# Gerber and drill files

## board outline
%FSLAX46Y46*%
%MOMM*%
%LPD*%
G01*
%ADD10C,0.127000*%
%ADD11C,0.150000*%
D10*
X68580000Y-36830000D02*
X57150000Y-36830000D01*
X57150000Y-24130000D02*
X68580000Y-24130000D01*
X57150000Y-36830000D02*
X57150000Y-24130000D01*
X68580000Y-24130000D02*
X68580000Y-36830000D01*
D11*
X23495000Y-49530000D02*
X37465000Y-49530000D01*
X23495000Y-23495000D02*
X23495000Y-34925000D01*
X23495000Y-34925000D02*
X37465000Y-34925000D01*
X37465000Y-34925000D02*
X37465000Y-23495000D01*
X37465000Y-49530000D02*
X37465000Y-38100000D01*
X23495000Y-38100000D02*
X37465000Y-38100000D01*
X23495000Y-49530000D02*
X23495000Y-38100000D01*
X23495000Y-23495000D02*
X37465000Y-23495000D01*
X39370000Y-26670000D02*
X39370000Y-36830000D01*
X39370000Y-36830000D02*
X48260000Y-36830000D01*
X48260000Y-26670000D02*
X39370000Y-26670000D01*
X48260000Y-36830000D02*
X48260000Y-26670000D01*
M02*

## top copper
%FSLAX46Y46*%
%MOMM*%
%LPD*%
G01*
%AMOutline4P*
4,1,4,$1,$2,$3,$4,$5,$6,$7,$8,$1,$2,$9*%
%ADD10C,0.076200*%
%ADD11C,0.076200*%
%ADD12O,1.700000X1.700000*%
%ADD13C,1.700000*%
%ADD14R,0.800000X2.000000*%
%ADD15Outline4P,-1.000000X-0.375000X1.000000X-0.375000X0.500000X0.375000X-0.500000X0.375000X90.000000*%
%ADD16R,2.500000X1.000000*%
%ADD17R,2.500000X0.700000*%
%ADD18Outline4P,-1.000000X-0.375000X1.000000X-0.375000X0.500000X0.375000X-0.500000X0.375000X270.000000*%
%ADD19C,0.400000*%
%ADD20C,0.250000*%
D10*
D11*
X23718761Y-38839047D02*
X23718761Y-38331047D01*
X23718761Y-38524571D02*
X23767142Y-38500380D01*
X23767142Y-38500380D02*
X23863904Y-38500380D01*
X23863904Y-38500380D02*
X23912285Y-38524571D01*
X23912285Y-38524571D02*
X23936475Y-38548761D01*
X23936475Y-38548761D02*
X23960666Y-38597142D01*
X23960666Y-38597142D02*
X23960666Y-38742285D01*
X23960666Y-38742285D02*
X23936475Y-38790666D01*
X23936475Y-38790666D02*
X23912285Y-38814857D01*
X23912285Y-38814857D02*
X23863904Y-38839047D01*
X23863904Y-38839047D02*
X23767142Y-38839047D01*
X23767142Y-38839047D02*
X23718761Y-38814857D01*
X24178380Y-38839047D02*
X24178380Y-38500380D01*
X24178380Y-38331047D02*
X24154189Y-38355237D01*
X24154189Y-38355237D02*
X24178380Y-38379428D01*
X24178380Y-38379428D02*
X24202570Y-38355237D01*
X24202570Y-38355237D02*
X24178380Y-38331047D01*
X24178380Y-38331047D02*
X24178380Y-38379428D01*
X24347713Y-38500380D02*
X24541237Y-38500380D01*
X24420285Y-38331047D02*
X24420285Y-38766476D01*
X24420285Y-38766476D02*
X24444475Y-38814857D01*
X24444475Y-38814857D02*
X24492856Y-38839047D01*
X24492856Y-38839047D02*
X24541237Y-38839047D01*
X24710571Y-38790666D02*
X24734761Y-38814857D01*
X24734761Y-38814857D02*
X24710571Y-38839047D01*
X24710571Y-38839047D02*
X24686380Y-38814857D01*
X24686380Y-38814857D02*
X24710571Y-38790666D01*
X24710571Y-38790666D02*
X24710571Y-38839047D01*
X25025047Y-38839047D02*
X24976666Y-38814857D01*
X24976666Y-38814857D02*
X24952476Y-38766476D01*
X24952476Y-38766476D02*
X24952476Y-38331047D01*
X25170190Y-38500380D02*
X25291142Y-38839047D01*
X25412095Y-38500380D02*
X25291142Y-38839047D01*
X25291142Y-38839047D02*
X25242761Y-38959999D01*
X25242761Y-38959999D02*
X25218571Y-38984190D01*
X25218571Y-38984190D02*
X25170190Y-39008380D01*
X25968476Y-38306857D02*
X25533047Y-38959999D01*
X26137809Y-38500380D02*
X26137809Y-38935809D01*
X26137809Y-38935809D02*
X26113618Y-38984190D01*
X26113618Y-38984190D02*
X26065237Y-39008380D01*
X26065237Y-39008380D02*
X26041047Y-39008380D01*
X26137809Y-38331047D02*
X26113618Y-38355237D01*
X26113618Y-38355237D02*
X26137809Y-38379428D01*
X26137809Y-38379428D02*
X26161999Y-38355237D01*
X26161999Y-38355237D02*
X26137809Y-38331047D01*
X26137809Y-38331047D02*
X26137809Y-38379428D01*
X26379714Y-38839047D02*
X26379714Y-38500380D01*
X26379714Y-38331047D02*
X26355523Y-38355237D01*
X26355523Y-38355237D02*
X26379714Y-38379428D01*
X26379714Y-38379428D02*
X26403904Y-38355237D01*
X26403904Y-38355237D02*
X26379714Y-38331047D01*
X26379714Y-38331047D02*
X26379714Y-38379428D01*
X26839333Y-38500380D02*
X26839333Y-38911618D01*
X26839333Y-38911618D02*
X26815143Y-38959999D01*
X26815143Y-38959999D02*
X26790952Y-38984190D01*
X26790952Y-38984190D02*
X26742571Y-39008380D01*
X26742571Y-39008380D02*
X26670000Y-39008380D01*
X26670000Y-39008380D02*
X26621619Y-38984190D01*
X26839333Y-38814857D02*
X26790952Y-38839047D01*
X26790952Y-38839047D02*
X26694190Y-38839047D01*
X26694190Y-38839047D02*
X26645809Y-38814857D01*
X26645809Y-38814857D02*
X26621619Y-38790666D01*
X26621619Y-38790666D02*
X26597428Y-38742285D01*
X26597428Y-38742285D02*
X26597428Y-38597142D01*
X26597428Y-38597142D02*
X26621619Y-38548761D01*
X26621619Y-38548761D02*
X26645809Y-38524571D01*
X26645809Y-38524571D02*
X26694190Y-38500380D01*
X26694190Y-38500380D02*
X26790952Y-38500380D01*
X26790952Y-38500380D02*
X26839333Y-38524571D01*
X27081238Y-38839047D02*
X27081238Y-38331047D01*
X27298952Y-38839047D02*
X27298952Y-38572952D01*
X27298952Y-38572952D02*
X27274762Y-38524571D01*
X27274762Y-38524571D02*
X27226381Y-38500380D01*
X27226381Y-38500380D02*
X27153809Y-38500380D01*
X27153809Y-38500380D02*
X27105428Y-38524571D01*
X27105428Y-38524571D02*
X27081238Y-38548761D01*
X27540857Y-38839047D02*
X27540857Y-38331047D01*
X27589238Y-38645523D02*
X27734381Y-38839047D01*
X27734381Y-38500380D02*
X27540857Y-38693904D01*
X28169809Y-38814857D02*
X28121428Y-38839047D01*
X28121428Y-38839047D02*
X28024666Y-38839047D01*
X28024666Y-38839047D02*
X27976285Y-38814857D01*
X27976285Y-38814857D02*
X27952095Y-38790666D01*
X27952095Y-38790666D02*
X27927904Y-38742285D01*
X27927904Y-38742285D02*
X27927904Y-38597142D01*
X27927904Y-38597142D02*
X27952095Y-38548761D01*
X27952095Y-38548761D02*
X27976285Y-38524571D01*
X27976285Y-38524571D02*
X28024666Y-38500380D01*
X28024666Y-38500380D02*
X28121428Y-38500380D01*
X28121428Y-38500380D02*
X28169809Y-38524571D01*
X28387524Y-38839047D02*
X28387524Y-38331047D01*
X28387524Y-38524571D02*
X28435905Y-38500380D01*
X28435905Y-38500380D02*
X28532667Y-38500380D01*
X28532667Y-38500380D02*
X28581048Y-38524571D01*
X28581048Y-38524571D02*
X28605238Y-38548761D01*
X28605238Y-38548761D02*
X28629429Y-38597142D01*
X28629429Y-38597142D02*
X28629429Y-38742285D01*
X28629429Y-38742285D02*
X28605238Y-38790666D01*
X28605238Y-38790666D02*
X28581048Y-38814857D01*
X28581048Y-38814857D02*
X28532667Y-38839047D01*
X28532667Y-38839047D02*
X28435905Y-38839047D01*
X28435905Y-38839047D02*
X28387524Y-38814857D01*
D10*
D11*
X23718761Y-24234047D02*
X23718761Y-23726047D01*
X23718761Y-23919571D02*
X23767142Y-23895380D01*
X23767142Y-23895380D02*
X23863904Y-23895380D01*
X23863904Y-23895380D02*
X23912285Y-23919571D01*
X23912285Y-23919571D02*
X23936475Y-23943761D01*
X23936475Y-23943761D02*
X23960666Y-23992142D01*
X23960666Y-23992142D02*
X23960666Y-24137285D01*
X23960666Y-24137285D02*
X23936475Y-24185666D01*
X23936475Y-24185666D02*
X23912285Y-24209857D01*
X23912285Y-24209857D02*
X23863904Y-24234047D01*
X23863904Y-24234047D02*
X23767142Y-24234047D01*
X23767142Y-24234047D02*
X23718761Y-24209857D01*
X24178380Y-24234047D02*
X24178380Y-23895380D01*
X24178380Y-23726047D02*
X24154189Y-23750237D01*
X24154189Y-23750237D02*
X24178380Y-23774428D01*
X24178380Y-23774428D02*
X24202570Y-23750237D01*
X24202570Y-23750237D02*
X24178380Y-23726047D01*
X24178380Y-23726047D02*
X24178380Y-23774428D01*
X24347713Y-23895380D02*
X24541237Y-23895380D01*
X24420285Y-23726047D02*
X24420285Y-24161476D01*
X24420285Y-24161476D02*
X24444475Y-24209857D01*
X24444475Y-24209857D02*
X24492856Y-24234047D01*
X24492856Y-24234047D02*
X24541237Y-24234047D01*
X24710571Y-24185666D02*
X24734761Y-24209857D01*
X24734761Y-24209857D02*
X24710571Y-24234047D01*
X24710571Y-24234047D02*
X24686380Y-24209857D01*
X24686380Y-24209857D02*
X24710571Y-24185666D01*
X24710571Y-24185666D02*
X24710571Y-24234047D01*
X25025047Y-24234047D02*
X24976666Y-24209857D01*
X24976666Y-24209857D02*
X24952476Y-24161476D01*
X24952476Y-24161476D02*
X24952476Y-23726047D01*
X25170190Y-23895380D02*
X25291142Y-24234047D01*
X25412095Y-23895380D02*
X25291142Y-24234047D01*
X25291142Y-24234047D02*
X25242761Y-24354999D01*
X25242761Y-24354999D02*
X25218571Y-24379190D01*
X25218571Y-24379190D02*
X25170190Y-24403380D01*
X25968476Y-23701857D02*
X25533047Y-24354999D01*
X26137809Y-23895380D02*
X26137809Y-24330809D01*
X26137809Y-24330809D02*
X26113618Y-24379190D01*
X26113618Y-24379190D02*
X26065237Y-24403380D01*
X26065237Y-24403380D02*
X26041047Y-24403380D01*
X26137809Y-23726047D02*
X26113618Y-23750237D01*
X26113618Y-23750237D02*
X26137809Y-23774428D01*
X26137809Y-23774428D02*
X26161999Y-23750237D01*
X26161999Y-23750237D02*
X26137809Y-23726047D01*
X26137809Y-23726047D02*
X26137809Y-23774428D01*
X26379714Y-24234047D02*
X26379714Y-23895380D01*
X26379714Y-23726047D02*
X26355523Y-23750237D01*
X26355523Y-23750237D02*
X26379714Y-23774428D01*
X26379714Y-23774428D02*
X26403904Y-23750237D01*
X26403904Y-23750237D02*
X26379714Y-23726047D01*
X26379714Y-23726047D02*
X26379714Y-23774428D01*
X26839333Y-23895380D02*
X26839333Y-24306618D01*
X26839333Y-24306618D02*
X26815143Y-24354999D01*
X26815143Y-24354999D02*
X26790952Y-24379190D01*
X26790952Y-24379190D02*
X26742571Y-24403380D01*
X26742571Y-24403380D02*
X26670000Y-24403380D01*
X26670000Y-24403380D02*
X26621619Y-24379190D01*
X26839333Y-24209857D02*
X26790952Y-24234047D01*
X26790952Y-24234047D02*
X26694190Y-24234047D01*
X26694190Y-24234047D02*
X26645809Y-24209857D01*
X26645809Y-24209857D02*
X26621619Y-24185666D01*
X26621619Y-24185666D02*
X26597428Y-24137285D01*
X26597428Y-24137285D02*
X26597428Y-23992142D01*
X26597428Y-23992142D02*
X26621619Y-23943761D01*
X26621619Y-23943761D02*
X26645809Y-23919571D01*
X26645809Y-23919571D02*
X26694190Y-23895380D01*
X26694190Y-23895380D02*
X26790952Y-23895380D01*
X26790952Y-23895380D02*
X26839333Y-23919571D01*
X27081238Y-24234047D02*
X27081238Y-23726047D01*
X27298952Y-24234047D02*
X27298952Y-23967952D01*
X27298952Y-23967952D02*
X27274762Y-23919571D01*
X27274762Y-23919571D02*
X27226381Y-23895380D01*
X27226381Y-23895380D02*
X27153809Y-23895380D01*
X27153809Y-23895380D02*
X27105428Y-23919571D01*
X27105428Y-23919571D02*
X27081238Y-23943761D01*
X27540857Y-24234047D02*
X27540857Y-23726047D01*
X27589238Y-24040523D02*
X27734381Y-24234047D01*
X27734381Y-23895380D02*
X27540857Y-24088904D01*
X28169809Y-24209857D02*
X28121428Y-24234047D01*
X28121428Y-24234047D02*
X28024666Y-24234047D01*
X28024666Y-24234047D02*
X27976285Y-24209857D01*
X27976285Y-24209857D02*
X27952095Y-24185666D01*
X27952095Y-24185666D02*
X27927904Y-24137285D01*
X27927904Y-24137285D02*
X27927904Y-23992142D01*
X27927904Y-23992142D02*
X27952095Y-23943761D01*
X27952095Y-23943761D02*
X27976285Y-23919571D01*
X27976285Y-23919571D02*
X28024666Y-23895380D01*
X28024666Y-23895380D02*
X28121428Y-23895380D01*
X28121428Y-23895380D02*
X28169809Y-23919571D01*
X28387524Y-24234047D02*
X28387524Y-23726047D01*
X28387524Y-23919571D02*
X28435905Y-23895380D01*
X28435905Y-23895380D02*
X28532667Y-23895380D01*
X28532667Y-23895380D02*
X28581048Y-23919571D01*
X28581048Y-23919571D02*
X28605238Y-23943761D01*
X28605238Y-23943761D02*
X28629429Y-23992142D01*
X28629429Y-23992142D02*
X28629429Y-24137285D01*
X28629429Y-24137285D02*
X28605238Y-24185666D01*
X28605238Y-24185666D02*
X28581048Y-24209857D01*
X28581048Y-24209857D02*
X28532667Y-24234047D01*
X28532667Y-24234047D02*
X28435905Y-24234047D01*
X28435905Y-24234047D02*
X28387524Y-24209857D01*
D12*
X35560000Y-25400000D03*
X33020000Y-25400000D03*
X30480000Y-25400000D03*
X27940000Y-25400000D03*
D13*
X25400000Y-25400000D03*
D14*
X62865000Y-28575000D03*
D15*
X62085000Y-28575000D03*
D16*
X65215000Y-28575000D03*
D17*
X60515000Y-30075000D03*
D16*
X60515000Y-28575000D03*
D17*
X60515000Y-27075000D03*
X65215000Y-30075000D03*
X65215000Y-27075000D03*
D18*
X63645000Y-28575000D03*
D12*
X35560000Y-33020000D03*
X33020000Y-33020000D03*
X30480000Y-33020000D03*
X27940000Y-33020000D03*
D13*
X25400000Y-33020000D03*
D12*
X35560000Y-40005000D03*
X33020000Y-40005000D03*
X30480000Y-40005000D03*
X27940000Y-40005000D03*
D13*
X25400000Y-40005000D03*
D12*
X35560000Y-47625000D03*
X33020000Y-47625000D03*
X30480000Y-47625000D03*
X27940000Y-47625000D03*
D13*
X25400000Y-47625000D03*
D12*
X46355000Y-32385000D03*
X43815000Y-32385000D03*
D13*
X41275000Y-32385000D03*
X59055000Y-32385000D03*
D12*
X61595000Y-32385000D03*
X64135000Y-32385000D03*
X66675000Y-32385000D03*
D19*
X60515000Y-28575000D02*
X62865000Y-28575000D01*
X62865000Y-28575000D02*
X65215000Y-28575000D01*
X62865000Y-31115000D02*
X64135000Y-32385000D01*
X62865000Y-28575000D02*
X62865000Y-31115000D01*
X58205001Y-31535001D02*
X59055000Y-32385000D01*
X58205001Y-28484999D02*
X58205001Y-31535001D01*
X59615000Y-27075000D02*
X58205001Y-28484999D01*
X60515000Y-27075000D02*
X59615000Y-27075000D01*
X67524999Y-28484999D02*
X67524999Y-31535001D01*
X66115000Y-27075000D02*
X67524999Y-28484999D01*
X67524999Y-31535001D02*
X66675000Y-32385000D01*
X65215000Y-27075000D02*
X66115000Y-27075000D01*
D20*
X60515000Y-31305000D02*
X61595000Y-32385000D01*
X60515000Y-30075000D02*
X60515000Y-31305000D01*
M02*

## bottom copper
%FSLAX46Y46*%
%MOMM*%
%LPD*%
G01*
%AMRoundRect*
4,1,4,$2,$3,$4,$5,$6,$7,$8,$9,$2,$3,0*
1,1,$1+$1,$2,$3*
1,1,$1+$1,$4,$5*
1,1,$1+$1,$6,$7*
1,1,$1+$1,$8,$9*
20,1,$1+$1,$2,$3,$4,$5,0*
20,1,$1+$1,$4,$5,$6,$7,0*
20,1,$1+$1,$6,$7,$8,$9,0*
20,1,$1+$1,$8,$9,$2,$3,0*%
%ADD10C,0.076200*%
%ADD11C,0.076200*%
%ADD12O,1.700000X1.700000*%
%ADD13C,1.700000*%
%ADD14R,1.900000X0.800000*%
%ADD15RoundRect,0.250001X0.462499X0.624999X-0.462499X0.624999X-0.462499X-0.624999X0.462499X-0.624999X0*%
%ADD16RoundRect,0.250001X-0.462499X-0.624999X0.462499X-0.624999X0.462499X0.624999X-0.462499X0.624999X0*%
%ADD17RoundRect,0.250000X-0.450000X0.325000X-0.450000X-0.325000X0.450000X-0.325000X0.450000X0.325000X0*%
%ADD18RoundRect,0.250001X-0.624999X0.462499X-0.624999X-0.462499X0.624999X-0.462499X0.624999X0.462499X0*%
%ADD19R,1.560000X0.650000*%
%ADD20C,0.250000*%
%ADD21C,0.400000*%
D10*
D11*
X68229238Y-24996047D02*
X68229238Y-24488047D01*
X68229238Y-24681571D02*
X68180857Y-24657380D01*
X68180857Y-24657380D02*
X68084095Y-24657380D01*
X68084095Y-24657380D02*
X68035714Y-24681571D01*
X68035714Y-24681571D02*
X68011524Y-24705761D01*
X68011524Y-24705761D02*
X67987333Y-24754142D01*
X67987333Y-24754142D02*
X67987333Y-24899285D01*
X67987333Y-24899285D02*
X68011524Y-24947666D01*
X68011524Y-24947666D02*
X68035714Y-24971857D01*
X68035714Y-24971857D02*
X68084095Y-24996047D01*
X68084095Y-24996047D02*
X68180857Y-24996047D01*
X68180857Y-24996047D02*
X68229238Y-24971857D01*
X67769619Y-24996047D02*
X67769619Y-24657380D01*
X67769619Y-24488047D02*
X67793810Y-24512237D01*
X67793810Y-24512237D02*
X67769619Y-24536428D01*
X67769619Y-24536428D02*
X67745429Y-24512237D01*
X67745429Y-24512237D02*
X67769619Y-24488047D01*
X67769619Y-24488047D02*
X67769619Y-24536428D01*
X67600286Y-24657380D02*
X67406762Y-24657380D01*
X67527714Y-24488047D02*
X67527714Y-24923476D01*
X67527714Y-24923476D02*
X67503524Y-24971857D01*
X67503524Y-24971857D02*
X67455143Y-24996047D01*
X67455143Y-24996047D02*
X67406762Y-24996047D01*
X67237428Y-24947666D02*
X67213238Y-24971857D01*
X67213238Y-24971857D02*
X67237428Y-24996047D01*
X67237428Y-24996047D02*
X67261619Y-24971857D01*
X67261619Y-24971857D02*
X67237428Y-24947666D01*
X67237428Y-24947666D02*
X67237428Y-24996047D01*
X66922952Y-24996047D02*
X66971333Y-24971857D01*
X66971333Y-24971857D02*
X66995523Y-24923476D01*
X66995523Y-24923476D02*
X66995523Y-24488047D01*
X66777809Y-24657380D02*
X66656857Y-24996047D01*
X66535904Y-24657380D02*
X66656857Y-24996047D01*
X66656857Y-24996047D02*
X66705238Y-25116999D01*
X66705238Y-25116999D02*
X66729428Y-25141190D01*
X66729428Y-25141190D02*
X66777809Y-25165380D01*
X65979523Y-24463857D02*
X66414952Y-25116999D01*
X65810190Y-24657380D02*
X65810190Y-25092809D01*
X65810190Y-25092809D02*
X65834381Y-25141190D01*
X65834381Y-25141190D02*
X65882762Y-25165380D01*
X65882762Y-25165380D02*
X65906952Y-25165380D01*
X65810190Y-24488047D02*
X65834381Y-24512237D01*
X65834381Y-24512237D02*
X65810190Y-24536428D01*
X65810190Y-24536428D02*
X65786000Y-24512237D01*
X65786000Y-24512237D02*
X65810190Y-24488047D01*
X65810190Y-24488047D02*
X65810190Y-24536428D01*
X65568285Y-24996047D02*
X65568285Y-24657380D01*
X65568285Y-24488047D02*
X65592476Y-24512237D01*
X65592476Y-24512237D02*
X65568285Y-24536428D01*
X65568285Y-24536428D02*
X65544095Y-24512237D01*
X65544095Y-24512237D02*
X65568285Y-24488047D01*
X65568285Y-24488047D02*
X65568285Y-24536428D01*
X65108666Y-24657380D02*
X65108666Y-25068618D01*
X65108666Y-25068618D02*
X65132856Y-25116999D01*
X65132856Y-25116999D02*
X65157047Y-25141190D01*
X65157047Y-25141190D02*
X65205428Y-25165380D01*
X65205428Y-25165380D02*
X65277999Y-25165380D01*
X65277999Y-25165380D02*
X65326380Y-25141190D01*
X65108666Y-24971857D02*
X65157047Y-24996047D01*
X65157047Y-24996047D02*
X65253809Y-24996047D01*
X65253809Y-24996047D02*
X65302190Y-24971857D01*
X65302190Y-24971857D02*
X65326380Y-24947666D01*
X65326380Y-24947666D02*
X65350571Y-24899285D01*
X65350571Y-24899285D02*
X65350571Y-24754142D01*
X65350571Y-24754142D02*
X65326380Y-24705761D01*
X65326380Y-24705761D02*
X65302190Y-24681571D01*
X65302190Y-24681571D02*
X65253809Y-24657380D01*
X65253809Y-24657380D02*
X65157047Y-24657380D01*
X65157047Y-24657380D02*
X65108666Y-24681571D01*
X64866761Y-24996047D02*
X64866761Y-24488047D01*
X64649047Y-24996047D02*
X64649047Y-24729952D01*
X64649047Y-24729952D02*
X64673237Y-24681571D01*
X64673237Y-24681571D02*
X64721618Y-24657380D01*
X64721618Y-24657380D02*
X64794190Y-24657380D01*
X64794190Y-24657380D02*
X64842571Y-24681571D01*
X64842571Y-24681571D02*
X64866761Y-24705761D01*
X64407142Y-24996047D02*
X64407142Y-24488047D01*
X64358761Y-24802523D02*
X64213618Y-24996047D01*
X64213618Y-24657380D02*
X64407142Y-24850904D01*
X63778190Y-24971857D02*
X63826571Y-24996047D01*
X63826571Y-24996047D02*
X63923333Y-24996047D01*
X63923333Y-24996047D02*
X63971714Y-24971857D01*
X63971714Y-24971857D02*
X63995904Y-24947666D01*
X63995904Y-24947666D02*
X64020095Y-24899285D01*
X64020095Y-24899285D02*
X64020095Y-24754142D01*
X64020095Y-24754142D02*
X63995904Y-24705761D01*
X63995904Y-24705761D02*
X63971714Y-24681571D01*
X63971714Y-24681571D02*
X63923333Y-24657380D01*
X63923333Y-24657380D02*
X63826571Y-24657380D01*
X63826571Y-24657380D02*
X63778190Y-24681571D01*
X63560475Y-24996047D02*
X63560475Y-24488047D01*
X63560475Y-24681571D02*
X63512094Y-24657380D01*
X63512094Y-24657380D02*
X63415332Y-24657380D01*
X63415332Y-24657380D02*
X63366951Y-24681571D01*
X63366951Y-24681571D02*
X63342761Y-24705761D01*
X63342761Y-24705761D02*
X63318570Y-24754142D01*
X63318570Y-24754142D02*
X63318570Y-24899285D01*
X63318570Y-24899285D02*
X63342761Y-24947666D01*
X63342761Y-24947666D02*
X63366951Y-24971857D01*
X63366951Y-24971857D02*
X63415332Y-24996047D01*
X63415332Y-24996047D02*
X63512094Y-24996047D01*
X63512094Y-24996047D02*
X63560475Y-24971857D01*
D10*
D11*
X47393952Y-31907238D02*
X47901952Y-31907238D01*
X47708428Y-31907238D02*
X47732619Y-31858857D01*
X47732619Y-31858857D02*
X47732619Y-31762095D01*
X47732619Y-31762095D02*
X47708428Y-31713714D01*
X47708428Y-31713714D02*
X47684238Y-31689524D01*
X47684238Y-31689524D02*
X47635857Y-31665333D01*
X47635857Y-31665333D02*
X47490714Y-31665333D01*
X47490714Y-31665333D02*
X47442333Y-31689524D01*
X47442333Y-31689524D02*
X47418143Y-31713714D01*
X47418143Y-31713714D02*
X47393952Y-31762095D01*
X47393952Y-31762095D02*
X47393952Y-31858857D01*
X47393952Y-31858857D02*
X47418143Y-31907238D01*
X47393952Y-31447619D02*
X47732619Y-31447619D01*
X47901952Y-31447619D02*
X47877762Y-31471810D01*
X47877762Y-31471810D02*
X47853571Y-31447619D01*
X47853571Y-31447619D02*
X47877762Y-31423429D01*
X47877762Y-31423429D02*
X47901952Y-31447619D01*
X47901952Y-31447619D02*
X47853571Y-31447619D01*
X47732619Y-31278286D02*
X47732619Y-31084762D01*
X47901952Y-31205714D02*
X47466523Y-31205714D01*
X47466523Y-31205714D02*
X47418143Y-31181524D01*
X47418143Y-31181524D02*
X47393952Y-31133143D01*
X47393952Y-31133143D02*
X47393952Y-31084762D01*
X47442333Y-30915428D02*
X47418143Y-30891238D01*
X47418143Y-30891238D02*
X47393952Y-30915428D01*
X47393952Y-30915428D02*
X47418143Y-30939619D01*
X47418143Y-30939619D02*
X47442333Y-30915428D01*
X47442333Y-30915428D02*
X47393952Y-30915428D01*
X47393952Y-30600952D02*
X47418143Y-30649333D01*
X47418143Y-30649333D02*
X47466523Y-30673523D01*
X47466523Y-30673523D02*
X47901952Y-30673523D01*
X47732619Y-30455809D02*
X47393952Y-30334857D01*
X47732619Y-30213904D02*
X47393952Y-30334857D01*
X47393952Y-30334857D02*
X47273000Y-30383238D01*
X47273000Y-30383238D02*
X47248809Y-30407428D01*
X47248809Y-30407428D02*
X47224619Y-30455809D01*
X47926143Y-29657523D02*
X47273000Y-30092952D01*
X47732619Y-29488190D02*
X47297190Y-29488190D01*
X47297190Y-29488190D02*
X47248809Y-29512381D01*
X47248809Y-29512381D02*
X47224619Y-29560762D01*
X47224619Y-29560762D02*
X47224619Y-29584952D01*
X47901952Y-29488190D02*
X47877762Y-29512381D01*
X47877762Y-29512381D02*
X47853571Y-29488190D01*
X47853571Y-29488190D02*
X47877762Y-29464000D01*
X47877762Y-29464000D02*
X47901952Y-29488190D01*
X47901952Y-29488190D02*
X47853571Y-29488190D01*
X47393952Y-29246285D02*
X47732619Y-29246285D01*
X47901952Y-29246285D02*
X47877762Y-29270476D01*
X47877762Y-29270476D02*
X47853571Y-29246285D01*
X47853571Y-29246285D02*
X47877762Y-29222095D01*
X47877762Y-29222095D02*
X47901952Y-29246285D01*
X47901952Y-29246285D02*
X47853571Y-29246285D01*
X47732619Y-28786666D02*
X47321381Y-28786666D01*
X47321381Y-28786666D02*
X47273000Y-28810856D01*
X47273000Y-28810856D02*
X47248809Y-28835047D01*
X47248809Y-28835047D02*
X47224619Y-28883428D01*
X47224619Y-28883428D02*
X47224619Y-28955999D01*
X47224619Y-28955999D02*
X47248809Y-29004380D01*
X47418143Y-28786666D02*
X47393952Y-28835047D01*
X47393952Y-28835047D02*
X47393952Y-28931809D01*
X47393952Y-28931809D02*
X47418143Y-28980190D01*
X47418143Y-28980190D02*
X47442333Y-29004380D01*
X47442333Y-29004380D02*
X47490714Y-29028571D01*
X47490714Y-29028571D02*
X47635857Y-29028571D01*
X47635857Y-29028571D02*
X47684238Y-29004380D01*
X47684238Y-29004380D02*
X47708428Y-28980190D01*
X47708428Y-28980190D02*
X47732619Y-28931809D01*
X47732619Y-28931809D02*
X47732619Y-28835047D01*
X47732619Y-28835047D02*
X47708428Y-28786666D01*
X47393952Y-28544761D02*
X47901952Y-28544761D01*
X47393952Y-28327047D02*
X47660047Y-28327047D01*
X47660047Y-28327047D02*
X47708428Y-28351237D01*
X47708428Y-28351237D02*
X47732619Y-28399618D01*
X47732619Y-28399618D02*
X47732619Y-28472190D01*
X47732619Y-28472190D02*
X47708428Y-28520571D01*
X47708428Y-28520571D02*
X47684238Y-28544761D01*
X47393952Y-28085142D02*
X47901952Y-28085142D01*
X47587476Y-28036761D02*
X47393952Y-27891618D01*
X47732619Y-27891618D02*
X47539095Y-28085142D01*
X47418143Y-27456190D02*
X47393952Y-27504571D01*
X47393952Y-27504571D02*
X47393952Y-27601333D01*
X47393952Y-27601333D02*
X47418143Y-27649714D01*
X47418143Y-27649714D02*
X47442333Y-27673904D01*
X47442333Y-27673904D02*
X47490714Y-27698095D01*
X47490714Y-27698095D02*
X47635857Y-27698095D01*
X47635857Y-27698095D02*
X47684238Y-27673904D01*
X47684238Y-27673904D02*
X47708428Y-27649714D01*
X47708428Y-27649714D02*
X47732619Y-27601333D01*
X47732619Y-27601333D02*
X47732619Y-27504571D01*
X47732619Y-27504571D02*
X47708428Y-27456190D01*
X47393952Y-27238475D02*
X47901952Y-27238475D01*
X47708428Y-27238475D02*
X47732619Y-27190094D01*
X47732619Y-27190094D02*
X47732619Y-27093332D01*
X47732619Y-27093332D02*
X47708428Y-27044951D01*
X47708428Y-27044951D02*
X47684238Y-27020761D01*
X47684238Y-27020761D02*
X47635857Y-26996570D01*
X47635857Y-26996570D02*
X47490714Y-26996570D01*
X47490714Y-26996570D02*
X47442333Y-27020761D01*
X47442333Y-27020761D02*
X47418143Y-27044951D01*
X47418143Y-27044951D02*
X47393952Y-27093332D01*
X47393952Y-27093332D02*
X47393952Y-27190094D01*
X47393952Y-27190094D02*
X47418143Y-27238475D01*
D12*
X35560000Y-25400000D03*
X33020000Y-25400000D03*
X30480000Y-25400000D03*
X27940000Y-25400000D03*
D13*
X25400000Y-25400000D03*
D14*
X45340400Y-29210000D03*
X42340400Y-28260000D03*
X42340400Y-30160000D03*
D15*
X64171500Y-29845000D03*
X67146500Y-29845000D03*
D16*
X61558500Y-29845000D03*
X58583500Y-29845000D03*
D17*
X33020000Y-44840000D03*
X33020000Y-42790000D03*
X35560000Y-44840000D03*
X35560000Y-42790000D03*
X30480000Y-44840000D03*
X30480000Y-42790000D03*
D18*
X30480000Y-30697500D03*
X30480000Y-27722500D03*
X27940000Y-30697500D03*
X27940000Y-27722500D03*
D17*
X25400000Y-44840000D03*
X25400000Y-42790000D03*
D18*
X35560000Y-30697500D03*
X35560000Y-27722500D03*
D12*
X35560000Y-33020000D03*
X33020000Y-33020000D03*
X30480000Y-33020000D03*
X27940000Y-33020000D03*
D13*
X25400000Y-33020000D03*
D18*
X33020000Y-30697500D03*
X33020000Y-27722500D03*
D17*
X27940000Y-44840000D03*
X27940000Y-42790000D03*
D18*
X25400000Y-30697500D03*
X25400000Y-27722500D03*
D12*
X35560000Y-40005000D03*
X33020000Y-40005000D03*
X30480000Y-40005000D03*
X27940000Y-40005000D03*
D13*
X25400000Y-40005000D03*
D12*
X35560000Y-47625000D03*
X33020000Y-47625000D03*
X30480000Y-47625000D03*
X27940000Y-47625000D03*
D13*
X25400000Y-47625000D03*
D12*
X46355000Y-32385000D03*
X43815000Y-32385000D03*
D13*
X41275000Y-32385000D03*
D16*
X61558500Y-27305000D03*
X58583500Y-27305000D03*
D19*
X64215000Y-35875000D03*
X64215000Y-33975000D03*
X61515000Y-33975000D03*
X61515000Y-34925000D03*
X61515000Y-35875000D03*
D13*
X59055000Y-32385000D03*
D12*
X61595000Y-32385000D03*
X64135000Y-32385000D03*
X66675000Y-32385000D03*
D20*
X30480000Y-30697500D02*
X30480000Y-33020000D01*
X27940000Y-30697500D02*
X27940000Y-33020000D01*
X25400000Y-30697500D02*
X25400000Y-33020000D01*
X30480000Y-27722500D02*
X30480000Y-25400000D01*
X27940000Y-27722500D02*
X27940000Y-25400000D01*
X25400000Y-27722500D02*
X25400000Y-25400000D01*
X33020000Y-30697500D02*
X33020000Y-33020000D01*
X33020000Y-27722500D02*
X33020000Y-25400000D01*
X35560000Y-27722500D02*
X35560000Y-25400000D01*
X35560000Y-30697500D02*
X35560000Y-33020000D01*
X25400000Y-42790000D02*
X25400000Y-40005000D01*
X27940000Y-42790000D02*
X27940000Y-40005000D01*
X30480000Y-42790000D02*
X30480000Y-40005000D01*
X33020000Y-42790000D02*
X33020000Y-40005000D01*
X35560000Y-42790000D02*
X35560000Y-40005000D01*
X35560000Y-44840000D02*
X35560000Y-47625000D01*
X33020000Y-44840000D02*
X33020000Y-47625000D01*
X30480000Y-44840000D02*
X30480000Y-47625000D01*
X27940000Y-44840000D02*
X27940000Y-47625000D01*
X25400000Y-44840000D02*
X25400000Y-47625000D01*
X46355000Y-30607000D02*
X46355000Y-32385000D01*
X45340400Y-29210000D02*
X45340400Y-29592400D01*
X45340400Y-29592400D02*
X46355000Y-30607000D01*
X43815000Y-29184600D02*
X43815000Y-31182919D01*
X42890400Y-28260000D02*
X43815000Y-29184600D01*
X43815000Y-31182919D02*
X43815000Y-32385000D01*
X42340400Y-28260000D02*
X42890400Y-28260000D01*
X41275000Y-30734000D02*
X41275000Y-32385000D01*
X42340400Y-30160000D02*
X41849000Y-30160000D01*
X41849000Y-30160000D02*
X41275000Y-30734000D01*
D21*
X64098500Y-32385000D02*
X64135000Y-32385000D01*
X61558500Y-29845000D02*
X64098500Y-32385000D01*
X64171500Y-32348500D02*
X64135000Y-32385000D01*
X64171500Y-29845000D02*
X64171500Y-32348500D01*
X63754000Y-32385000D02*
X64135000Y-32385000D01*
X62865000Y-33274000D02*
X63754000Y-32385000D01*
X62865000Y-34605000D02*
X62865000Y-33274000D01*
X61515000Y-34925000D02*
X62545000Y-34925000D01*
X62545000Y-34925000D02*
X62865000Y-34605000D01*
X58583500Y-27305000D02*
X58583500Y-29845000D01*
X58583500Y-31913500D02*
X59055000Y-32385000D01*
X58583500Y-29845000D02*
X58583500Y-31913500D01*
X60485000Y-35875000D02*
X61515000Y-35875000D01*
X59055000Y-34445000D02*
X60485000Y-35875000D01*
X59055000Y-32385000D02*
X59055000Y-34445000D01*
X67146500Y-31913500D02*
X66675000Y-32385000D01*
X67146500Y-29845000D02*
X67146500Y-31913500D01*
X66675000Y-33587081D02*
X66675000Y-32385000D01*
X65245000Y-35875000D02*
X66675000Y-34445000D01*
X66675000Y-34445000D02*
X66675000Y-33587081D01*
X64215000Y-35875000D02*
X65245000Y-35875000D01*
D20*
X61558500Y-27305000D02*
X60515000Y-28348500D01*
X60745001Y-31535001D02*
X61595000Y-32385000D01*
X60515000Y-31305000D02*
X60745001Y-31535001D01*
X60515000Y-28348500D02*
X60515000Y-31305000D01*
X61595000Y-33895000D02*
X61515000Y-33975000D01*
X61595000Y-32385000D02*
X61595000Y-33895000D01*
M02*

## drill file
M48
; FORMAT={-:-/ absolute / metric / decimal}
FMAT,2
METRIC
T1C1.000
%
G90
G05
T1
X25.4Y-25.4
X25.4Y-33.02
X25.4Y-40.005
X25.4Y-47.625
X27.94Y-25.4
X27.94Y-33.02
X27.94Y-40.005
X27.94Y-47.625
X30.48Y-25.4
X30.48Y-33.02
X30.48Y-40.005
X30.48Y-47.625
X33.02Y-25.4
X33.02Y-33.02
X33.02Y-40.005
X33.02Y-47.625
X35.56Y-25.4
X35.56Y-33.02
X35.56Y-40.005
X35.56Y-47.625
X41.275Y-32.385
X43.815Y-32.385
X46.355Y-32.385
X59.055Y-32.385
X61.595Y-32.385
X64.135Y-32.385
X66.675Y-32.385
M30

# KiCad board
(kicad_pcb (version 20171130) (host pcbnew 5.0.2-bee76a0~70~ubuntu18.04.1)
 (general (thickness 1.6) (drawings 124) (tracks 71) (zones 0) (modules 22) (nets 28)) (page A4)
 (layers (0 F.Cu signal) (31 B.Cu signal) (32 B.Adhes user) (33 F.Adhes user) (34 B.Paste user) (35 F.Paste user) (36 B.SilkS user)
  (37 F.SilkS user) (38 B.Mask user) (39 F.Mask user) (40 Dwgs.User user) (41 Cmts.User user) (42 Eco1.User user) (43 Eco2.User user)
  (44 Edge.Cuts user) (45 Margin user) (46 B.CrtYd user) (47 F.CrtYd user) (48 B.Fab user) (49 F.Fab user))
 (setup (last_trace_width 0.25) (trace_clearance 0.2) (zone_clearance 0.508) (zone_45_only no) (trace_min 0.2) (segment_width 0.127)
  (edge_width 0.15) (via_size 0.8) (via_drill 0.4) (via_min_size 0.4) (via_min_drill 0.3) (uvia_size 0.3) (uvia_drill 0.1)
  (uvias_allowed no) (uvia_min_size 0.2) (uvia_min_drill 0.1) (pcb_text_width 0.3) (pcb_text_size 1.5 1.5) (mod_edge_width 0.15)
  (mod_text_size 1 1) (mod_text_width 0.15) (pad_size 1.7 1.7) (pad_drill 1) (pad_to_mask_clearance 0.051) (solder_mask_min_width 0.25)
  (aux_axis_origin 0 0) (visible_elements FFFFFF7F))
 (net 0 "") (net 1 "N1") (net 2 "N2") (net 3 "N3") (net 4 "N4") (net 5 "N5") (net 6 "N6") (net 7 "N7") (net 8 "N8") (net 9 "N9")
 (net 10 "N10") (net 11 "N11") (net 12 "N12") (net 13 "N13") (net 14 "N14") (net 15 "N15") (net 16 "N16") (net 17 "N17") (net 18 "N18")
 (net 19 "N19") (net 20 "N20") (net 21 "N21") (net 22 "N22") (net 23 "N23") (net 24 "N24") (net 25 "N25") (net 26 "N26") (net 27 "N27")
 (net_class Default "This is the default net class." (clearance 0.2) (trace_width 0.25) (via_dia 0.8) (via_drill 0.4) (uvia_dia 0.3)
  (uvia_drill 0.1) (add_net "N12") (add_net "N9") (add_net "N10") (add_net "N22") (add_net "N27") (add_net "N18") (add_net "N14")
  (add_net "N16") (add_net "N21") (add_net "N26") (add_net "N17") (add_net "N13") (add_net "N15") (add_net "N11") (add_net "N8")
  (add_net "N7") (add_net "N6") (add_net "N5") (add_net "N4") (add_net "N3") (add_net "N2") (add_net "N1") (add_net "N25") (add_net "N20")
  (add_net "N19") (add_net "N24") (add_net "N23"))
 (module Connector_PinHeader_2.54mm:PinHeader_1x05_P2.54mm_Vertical (layer B.Cu) (at 25.4 25.4 270)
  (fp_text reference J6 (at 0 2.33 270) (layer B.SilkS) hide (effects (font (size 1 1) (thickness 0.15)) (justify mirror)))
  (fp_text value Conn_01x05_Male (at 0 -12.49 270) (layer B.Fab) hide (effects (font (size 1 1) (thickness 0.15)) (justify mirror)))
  (pad 5 thru_hole oval (at 0 -10.16 270) (size 1.7 1.7) (drill 1) (layers *.Cu *.Mask) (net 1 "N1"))
  (pad 4 thru_hole oval (at 0 -7.62 270) (size 1.7 1.7) (drill 1) (layers *.Cu *.Mask) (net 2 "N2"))
  (pad 3 thru_hole oval (at 0 -5.08 270) (size 1.7 1.7) (drill 1) (layers *.Cu *.Mask) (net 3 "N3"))
  (pad 2 thru_hole oval (at 0 -2.54 270) (size 1.7 1.7) (drill 1) (layers *.Cu *.Mask) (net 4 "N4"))
  (pad 1 thru_hole circle (at 0 0 270) (size 1.7 1.7) (drill 1) (layers *.Cu *.Mask) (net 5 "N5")))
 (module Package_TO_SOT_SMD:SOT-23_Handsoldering (layer B.Cu) (at 43.8404 29.21)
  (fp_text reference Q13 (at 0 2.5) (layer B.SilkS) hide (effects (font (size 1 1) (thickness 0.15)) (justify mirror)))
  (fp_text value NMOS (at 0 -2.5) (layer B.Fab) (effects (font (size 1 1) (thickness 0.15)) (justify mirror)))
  (pad 3 smd rect (at 1.5 0) (size 1.9 0.8) (layers B.Cu B.Paste B.Mask) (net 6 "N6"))
  (pad 2 smd rect (at -1.5 -0.95) (size 1.9 0.8) (layers B.Cu B.Paste B.Mask) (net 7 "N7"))
  (pad 1 smd rect (at -1.5 0.95) (size 1.9 0.8) (layers B.Cu B.Paste B.Mask) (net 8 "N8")))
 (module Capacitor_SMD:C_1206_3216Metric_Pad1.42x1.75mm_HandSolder (layer B.Cu) (at 65.659 29.845 180)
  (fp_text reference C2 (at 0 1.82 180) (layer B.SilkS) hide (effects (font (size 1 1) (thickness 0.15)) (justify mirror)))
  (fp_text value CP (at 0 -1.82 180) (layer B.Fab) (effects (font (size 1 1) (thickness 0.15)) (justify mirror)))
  (pad 2 smd roundrect (at 1.4875 0 180) (size 1.425 1.75) (layers B.Cu B.Paste B.Mask) (roundrect_rratio 0.175439) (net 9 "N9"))
  (pad 1 smd roundrect (at -1.4875 0 180) (size 1.425 1.75) (layers B.Cu B.Paste B.Mask) (roundrect_rratio 0.175439) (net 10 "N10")))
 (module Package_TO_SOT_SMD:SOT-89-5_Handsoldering (layer F.Cu) (at 62.865 28.575)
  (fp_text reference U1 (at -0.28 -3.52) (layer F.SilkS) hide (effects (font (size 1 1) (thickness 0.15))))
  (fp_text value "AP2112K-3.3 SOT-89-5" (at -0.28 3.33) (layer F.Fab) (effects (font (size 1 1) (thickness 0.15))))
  (pad 2 smd rect (at 0 0 270) (size 2 0.8) (layers F.Cu F.Paste F.Mask) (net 9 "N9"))
  (pad 2 smd trapezoid (at -0.78 0 90) (size 1.5 0.75) (rect_delta 0 0.5) (layers F.Cu F.Paste F.Mask) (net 9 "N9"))
  (pad 2 smd rect (at 2.35 0 270) (size 1 2.5) (layers F.Cu F.Paste F.Mask) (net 9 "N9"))
  (pad 3 smd rect (at -2.35 1.5 270) (size 0.7 2.5) (layers F.Cu F.Paste F.Mask) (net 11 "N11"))
  (pad 2 smd rect (at -2.35 0 270) (size 1 2.5) (layers F.Cu F.Paste F.Mask) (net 9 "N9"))
  (pad 1 smd rect (at -2.35 -1.5 270) (size 0.7 2.5) (layers F.Cu F.Paste F.Mask) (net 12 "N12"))
  (pad 4 smd rect (at 2.35 1.5 270) (size 0.7 2.5) (layers F.Cu F.Paste F.Mask))
  (pad 5 smd rect (at 2.35 -1.5 270) (size 0.7 2.5) (layers F.Cu F.Paste F.Mask) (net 10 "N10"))
  (pad 2 smd trapezoid (at 0.78 0 270) (size 1.5 0.75) (rect_delta 0 0.5) (layers F.Cu F.Paste F.Mask) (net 9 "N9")))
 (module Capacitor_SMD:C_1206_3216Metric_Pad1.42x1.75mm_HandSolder (layer B.Cu) (at 60.071 29.845)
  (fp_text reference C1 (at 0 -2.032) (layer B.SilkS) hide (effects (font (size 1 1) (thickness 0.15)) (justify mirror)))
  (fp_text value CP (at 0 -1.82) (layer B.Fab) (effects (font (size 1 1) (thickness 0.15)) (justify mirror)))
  (pad 2 smd roundrect (at 1.4875 0) (size 1.425 1.75) (layers B.Cu B.Paste B.Mask) (roundrect_rratio 0.175439) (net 9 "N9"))
  (pad 1 smd roundrect (at -1.4875 0) (size 1.425 1.75) (layers B.Cu B.Paste B.Mask) (roundrect_rratio 0.175439) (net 12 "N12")))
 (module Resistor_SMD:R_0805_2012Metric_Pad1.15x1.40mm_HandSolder (layer B.Cu) (at 33.02 43.815 270)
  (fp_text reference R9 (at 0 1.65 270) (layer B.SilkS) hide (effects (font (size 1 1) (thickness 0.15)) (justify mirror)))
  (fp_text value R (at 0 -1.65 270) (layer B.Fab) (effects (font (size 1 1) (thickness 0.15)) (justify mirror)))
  (pad 2 smd roundrect (at 1.025 0 270) (size 1.15 1.4) (layers B.Cu B.Paste B.Mask) (roundrect_rratio 0.217391) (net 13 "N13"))
  (pad 1 smd roundrect (at -1.025 0 270) (size 1.15 1.4) (layers B.Cu B.Paste B.Mask) (roundrect_rratio 0.217391) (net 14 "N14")))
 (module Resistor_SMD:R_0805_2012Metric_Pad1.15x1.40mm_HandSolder (layer B.Cu) (at 35.56 43.815 270)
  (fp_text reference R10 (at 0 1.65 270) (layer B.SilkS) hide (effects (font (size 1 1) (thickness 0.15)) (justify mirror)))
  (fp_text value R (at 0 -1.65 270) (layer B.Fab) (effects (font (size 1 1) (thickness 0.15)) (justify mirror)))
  (pad 2 smd roundrect (at 1.025 0 270) (size 1.15 1.4) (layers B.Cu B.Paste B.Mask) (roundrect_rratio 0.217391) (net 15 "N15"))
  (pad 1 smd roundrect (at -1.025 0 270) (size 1.15 1.4) (layers B.Cu B.Paste B.Mask) (roundrect_rratio 0.217391) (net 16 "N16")))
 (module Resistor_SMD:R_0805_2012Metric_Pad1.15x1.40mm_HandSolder (layer B.Cu) (at 30.48 43.815 270)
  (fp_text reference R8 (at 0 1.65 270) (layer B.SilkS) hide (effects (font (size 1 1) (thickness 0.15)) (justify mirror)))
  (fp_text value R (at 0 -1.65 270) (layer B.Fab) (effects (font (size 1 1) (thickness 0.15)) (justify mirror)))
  (pad 2 smd roundrect (at 1.025 0 270) (size 1.15 1.4) (layers B.Cu B.Paste B.Mask) (roundrect_rratio 0.217391) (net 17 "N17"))
  (pad 1 smd roundrect (at -1.025 0 270) (size 1.15 1.4) (layers B.Cu B.Paste B.Mask) (roundrect_rratio 0.217391) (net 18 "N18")))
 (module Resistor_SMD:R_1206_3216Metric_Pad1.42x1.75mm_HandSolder (layer B.Cu) (at 30.48 29.21 270)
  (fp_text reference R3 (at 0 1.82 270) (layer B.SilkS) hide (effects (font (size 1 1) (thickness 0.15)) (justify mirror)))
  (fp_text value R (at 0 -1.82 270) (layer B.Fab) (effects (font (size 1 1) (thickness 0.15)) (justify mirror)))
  (pad 2 smd roundrect (at 1.4875 0 270) (size 1.425 1.75) (layers B.Cu B.Paste B.Mask) (roundrect_rratio 0.175439) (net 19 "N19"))
  (pad 1 smd roundrect (at -1.4875 0 270) (size 1.425 1.75) (layers B.Cu B.Paste B.Mask) (roundrect_rratio 0.175439) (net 3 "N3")))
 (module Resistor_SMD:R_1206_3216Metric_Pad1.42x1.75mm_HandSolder (layer B.Cu) (at 27.94 29.21 270)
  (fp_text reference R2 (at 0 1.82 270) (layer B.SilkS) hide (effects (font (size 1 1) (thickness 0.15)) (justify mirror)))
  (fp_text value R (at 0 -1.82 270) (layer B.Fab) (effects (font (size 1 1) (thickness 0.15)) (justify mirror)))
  (pad 2 smd roundrect (at 1.4875 0 270) (size 1.425 1.75) (layers B.Cu B.Paste B.Mask) (roundrect_rratio 0.175439) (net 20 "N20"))
  (pad 1 smd roundrect (at -1.4875 0 270) (size 1.425 1.75) (layers B.Cu B.Paste B.Mask) (roundrect_rratio 0.175439) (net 4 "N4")))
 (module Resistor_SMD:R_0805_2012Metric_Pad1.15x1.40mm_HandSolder (layer B.Cu) (at 25.4 43.815 270)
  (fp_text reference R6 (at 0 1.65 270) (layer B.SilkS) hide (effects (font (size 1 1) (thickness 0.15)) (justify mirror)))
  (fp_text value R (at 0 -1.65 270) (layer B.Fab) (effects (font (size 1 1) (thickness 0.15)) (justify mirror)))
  (pad 2 smd roundrect (at 1.025 0 270) (size 1.15 1.4) (layers B.Cu B.Paste B.Mask) (roundrect_rratio 0.217391) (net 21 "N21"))
  (pad 1 smd roundrect (at -1.025 0 270) (size 1.15 1.4) (layers B.Cu B.Paste B.Mask) (roundrect_rratio 0.217391) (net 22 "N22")))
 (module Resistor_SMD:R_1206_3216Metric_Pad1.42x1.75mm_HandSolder (layer B.Cu) (at 35.56 29.21 270)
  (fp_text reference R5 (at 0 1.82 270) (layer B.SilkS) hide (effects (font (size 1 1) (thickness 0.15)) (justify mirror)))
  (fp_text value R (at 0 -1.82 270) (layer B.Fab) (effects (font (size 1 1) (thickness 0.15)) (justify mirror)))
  (pad 2 smd roundrect (at 1.4875 0 270) (size 1.425 1.75) (layers B.Cu B.Paste B.Mask) (roundrect_rratio 0.175439) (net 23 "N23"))
  (pad 1 smd roundrect (at -1.4875 0 270) (size 1.425 1.75) (layers B.Cu B.Paste B.Mask) (roundrect_rratio 0.175439) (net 1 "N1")))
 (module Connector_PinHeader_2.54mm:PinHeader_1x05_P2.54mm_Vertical (layer B.Cu) (at 25.4 33.02 270)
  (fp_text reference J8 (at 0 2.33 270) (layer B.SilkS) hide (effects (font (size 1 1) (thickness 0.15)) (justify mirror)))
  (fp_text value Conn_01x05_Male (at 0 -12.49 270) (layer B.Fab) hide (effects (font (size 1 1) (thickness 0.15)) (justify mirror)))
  (pad 5 thru_hole oval (at 0 -10.16 270) (size 1.7 1.7) (drill 1) (layers *.Cu *.Mask) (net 23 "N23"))
  (pad 4 thru_hole oval (at 0 -7.62 270) (size 1.7 1.7) (drill 1) (layers *.Cu *.Mask) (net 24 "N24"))
  (pad 3 thru_hole oval (at 0 -5.08 270) (size 1.7 1.7) (drill 1) (layers *.Cu *.Mask) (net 19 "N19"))
  (pad 2 thru_hole oval (at 0 -2.54 270) (size 1.7 1.7) (drill 1) (layers *.Cu *.Mask) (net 20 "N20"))
  (pad 1 thru_hole circle (at 0 0 270) (size 1.7 1.7) (drill 1) (layers *.Cu *.Mask) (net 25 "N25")))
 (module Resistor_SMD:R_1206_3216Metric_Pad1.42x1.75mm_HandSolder (layer B.Cu) (at 33.02 29.21 270)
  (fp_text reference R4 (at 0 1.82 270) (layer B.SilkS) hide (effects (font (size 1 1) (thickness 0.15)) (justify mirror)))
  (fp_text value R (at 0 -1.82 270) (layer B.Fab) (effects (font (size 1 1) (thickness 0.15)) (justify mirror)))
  (pad 2 smd roundrect (at 1.4875 0 270) (size 1.425 1.75) (layers B.Cu B.Paste B.Mask) (roundrect_rratio 0.175439) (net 24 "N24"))
  (pad 1 smd roundrect (at -1.4875 0 270) (size 1.425 1.75) (layers B.Cu B.Paste B.Mask) (roundrect_rratio 0.175439) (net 2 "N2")))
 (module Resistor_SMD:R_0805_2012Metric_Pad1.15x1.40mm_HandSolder (layer B.Cu) (at 27.94 43.815 270)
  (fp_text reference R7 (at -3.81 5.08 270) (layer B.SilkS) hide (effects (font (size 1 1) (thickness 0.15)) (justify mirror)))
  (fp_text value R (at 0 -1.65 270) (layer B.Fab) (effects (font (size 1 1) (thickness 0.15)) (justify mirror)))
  (pad 2 smd roundrect (at 1.025 0 270) (size 1.15 1.4) (layers B.Cu B.Paste B.Mask) (roundrect_rratio 0.217391) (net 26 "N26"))
  (pad 1 smd roundrect (at -1.025 0 270) (size 1.15 1.4) (layers B.Cu B.Paste B.Mask) (roundrect_rratio 0.217391) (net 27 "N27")))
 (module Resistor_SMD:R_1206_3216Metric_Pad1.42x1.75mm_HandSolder (layer B.Cu) (at 25.4 29.21 270)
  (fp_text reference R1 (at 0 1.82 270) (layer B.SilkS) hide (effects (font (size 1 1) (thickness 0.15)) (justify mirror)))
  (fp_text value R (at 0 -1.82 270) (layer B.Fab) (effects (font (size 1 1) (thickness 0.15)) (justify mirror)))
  (pad 2 smd roundrect (at 1.4875 0 270) (size 1.425 1.75) (layers B.Cu B.Paste B.Mask) (roundrect_rratio 0.175439) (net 25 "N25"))
  (pad 1 smd roundrect (at -1.4875 0 270) (size 1.425 1.75) (layers B.Cu B.Paste B.Mask) (roundrect_rratio 0.175439) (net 5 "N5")))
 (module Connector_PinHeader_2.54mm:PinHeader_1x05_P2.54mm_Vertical (layer B.Cu) (at 25.4 40.005 270)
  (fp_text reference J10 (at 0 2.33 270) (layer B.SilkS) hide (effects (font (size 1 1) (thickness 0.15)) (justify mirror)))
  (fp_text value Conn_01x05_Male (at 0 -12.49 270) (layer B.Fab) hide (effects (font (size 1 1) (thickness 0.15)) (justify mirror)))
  (pad 5 thru_hole oval (at 0 -10.16 270) (size 1.7 1.7) (drill 1) (layers *.Cu *.Mask) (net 16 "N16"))
  (pad 4 thru_hole oval (at 0 -7.62 270) (size 1.7 1.7) (drill 1) (layers *.Cu *.Mask) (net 14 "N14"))
  (pad 3 thru_hole oval (at 0 -5.08 270) (size 1.7 1.7) (drill 1) (layers *.Cu *.Mask) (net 18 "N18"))
  (pad 2 thru_hole oval (at 0 -2.54 270) (size 1.7 1.7) (drill 1) (layers *.Cu *.Mask) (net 27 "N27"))
  (pad 1 thru_hole circle (at 0 0 270) (size 1.7 1.7) (drill 1) (layers *.Cu *.Mask) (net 22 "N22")))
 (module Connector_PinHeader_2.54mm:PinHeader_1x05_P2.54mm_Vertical (layer B.Cu) (at 25.4 47.625 270)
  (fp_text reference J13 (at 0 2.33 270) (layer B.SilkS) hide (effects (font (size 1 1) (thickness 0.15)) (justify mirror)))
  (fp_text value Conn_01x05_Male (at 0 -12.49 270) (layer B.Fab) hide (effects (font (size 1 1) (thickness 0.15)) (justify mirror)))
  (pad 5 thru_hole oval (at 0 -10.16 270) (size 1.7 1.7) (drill 1) (layers *.Cu *.Mask) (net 15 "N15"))
  (pad 4 thru_hole oval (at 0 -7.62 270) (size 1.7 1.7) (drill 1) (layers *.Cu *.Mask) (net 13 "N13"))
  (pad 3 thru_hole oval (at 0 -5.08 270) (size 1.7 1.7) (drill 1) (layers *.Cu *.Mask) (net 17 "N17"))
  (pad 2 thru_hole oval (at 0 -2.54 270) (size 1.7 1.7) (drill 1) (layers *.Cu *.Mask) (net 26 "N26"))
  (pad 1 thru_hole circle (at 0 0 270) (size 1.7 1.7) (drill 1) (layers *.Cu *.Mask) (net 21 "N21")))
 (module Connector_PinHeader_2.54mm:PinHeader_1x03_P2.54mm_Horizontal (layer B.Cu) (at 41.275 32.385 270)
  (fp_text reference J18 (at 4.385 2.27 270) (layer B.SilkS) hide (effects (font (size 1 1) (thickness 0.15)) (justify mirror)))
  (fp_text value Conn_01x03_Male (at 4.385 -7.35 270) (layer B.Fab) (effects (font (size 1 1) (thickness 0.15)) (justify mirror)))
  (pad 3 thru_hole oval (at 0 -5.08 270) (size 1.7 1.7) (drill 1) (layers *.Cu *.Mask) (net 6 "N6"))
  (pad 2 thru_hole oval (at 0 -2.54 270) (size 1.7 1.7) (drill 1) (layers *.Cu *.Mask) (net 7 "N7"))
  (pad 1 thru_hole circle (at 0 0 270) (size 1.7 1.7) (drill 1) (layers *.Cu *.Mask) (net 8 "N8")))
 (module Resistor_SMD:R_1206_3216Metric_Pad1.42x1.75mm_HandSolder (layer B.Cu) (at 60.071 27.305)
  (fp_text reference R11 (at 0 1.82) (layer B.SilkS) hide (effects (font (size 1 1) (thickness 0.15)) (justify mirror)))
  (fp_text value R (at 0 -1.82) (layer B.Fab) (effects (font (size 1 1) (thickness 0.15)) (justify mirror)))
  (pad 2 smd roundrect (at 1.4875 0) (size 1.425 1.75) (layers B.Cu B.Paste B.Mask) (roundrect_rratio 0.175439) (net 11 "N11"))
  (pad 1 smd roundrect (at -1.4875 0) (size 1.425 1.75) (layers B.Cu B.Paste B.Mask) (roundrect_rratio 0.175439) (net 12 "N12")))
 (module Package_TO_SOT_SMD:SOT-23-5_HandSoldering (layer B.Cu) (at 62.865 34.925)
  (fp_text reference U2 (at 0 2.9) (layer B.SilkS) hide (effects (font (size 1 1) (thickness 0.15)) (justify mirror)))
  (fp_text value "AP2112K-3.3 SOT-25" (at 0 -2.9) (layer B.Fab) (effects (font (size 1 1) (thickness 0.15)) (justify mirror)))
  (pad 5 smd rect (at 1.35 0.95) (size 1.56 0.65) (layers B.Cu B.Paste B.Mask) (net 10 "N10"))
  (pad 4 smd rect (at 1.35 -0.95) (size 1.56 0.65) (layers B.Cu B.Paste B.Mask))
  (pad 3 smd rect (at -1.35 -0.95) (size 1.56 0.65) (layers B.Cu B.Paste B.Mask) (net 11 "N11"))
  (pad 2 smd rect (at -1.35 0) (size 1.56 0.65) (layers B.Cu B.Paste B.Mask) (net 9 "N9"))
  (pad 1 smd rect (at -1.35 0.95) (size 1.56 0.65) (layers B.Cu B.Paste B.Mask) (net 12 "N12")))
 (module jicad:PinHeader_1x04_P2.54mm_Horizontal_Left (layer F.Cu) (at 59.055 32.385 90)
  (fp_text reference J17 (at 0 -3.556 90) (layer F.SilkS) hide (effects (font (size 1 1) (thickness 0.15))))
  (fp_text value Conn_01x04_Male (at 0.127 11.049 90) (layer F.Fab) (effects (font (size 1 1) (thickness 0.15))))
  (pad 1 thru_hole circle (at 0 0 90) (size 1.7 1.7) (drill 1) (layers *.Cu *.Mask) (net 12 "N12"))
  (pad 2 thru_hole oval (at 0 2.54 90) (size 1.7 1.7) (drill 1) (layers *.Cu *.Mask) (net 11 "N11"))
  (pad 3 thru_hole oval (at 0 5.08 90) (size 1.7 1.7) (drill 1) (layers *.Cu *.Mask) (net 9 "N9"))
  (pad 4 thru_hole oval (at 0 7.62 90) (size 1.7 1.7) (drill 1) (layers *.Cu *.Mask) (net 10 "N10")))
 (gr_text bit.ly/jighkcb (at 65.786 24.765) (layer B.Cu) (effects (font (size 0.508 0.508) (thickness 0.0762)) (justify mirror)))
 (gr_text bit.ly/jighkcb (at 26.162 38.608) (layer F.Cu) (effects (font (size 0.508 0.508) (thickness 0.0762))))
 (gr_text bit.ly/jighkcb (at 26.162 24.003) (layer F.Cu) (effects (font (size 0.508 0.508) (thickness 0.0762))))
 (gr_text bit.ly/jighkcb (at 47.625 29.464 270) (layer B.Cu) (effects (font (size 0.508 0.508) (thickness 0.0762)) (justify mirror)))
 (gr_line (start 68.58 36.83) (end 57.15 36.83) (layer Edge.Cuts) (width 0.127))
 (gr_line (start 57.15 24.13) (end 68.58 24.13) (layer Edge.Cuts) (width 0.127))
 (gr_line (start 57.15 36.83) (end 57.15 24.13) (layer Edge.Cuts) (width 0.127))
 (gr_line (start 68.58 24.13) (end 68.58 36.83) (layer Edge.Cuts) (width 0.127))
 (gr_line (start 23.495 49.53) (end 37.465 49.53) (layer Edge.Cuts) (width 0.15))
 (gr_line (start 23.495 23.495) (end 23.495 34.925) (layer Edge.Cuts) (width 0.15))
 (gr_line (start 23.495 34.925) (end 37.465 34.925) (layer Edge.Cuts) (width 0.15))
 (gr_line (start 37.465 34.925) (end 37.465 23.495) (layer Edge.Cuts) (width 0.15))
 (gr_line (start 37.465 49.53) (end 37.465 38.1) (layer Edge.Cuts) (width 0.15))
 (gr_line (start 23.495 38.1) (end 37.465 38.1) (layer Edge.Cuts) (width 0.15))
 (gr_line (start 23.495 49.53) (end 23.495 38.1) (layer Edge.Cuts) (width 0.15))
 (gr_line (start 23.495 23.495) (end 37.465 23.495) (layer Edge.Cuts) (width 0.15))
 (gr_line (start 39.37 26.67) (end 39.37 36.83) (layer Edge.Cuts) (width 0.15))
 (gr_line (start 39.37 36.83) (end 48.26 36.83) (layer Edge.Cuts) (width 0.15))
 (gr_line (start 48.26 26.67) (end 39.37 26.67) (layer Edge.Cuts) (width 0.15))
 (gr_line (start 48.26 36.83) (end 48.26 26.67) (layer Edge.Cuts) (width 0.15))
 (segment (start 30.48 30.6975) (end 30.48 33.02) (width 0.25) (layer B.Cu) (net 19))
 (segment (start 27.94 30.6975) (end 27.94 33.02) (width 0.25) (layer B.Cu) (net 20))
 (segment (start 25.4 30.6975) (end 25.4 33.02) (width 0.25) (layer B.Cu) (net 25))
 (segment (start 30.48 27.7225) (end 30.48 25.4) (width 0.25) (layer B.Cu) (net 3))
 (segment (start 27.94 27.7225) (end 27.94 25.4) (width 0.25) (layer B.Cu) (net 4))
 (segment (start 25.4 27.7225) (end 25.4 25.4) (width 0.25) (layer B.Cu) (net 5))
 (segment (start 33.02 30.6975) (end 33.02 33.02) (width 0.25) (layer B.Cu) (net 24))
 (segment (start 33.02 27.7225) (end 33.02 25.4) (width 0.25) (layer B.Cu) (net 2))
 (segment (start 35.56 27.7225) (end 35.56 25.4) (width 0.25) (layer B.Cu) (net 1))
 (segment (start 35.56 30.6975) (end 35.56 33.02) (width 0.25) (layer B.Cu) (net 23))
 (segment (start 25.4 42.79) (end 25.4 40.005) (width 0.25) (layer B.Cu) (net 22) (status 30))
 (segment (start 27.94 42.79) (end 27.94 40.005) (width 0.25) (layer B.Cu) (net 27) (status 30))
 (segment (start 30.48 42.79) (end 30.48 40.005) (width 0.25) (layer B.Cu) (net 18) (status 30))
 (segment (start 33.02 42.79) (end 33.02 40.005) (width 0.25) (layer B.Cu) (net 14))
 (segment (start 35.56 42.79) (end 35.56 40.005) (width 0.25) (layer B.Cu) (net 16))
 (segment (start 35.56 44.84) (end 35.56 47.625) (width 0.25) (layer B.Cu) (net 15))
 (segment (start 33.02 44.84) (end 33.02 47.625) (width 0.25) (layer B.Cu) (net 13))
 (segment (start 30.48 44.84) (end 30.48 47.625) (width 0.25) (layer B.Cu) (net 17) (status 30))
 (segment (start 27.94 44.84) (end 27.94 47.625) (width 0.25) (layer B.Cu) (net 26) (status 30))
 (segment (start 25.4 44.84) (end 25.4 47.625) (width 0.25) (layer B.Cu) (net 21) (status 30))
 (segment (start 46.355 30.607) (end 46.355 32.385) (width 0.25) (layer B.Cu) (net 6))
 (segment (start 45.3404 29.21) (end 45.3404 29.5924) (width 0.25) (layer B.Cu) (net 6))
 (segment (start 45.3404 29.5924) (end 46.355 30.607) (width 0.25) (layer B.Cu) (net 6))
 (segment (start 43.815 29.1846) (end 43.815 31.182919) (width 0.25) (layer B.Cu) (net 7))
 (segment (start 42.8904 28.26) (end 43.815 29.1846) (width 0.25) (layer B.Cu) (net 7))
 (segment (start 43.815 31.182919) (end 43.815 32.385) (width 0.25) (layer B.Cu) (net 7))
 (segment (start 42.3404 28.26) (end 42.8904 28.26) (width 0.25) (layer B.Cu) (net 7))
 (segment (start 41.275 30.734) (end 41.275 32.385) (width 0.25) (layer B.Cu) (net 8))
 (segment (start 42.3404 30.16) (end 41.849 30.16) (width 0.25) (layer B.Cu) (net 8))
 (segment (start 41.849 30.16) (end 41.275 30.734) (width 0.25) (layer B.Cu) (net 8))
 (segment (start 60.515 28.575) (end 62.865 28.575) (width 0.4) (layer F.Cu) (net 9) (status 30))
 (segment (start 62.865 28.575) (end 65.215 28.575) (width 0.4) (layer F.Cu) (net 9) (status 30))
 (segment (start 62.865 31.115) (end 64.135 32.385) (width 0.4) (layer F.Cu) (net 9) (status 20))
 (segment (start 62.865 28.575) (end 62.865 31.115) (width 0.4) (layer F.Cu) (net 9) (status 10))
 (segment (start 64.0985 32.385) (end 64.135 32.385) (width 0.4) (layer B.Cu) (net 9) (status 30))
 (segment (start 61.5585 29.845) (end 64.0985 32.385) (width 0.4) (layer B.Cu) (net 9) (status 30))
 (segment (start 64.1715 32.3485) (end 64.135 32.385) (width 0.4) (layer B.Cu) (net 9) (status 30))
 (segment (start 64.1715 29.845) (end 64.1715 32.3485) (width 0.4) (layer B.Cu) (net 9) (status 30))
 (segment (start 63.754 32.385) (end 64.135 32.385) (width 0.4) (layer B.Cu) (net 9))
 (segment (start 62.865 33.274) (end 63.754 32.385) (width 0.4) (layer B.Cu) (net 9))
 (segment (start 62.865 34.605) (end 62.865 33.274) (width 0.4) (layer B.Cu) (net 9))
 (segment (start 61.515 34.925) (end 62.545 34.925) (width 0.4) (layer B.Cu) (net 9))
 (segment (start 62.545 34.925) (end 62.865 34.605) (width 0.4) (layer B.Cu) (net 9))
 (segment (start 58.5835 27.305) (end 58.5835 29.845) (width 0.4) (layer B.Cu) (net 12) (status 30))
 (segment (start 58.5835 31.9135) (end 59.055 32.385) (width 0.4) (layer B.Cu) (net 12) (status 30))
 (segment (start 58.5835 29.845) (end 58.5835 31.9135) (width 0.4) (layer B.Cu) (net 12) (status 30))
 (segment (start 60.485 35.875) (end 61.515 35.875) (width 0.4) (layer B.Cu) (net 12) (status 20))
 (segment (start 59.055 34.445) (end 60.485 35.875) (width 0.4) (layer B.Cu) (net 12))
 (segment (start 59.055 32.385) (end 59.055 34.445) (width 0.4) (layer B.Cu) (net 12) (status 10))
 (segment (start 58.205001 31.535001) (end 59.055 32.385) (width 0.4) (layer F.Cu) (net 12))
 (segment (start 58.205001 28.484999) (end 58.205001 31.535001) (width 0.4) (layer F.Cu) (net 12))
 (segment (start 59.615 27.075) (end 58.205001 28.484999) (width 0.4) (layer F.Cu) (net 12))
 (segment (start 60.515 27.075) (end 59.615 27.075) (width 0.4) (layer F.Cu) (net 12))
 (segment (start 67.1465 31.9135) (end 66.675 32.385) (width 0.4) (layer B.Cu) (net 10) (status 30))
 (segment (start 67.1465 29.845) (end 67.1465 31.9135) (width 0.4) (layer B.Cu) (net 10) (status 30))
 (segment (start 66.675 33.587081) (end 66.675 32.385) (width 0.4) (layer B.Cu) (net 10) (status 20))
 (segment (start 65.245 35.875) (end 66.675 34.445) (width 0.4) (layer B.Cu) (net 10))
 (segment (start 66.675 34.445) (end 66.675 33.587081) (width 0.4) (layer B.Cu) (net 10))
 (segment (start 64.215 35.875) (end 65.245 35.875) (width 0.4) (layer B.Cu) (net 10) (status 10))
 (segment (start 67.524999 28.484999) (end 67.524999 31.535001) (width 0.4) (layer F.Cu) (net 10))
 (segment (start 66.115 27.075) (end 67.524999 28.484999) (width 0.4) (layer F.Cu) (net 10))
 (segment (start 67.524999 31.535001) (end 66.675 32.385) (width 0.4) (layer F.Cu) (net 10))
 (segment (start 65.215 27.075) (end 66.115 27.075) (width 0.4) (layer F.Cu) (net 10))
 (segment (start 60.515 31.305) (end 61.595 32.385) (width 0.25) (layer F.Cu) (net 11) (status 20))
 (segment (start 60.515 30.075) (end 60.515 31.305) (width 0.25) (layer F.Cu) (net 11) (status 10))
 (segment (start 61.5585 27.305) (end 60.515 28.3485) (width 0.25) (layer B.Cu) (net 11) (status 10))
 (segment (start 60.745001 31.535001) (end 61.595 32.385) (width 0.25) (layer B.Cu) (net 11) (status 30))
 (segment (start 60.515 31.305) (end 60.745001 31.535001) (width 0.25) (layer B.Cu) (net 11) (status 20))
 (segment (start 60.515 28.3485) (end 60.515 31.305) (width 0.25) (layer B.Cu) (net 11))
 (segment (start 61.595 33.895) (end 61.515 33.975) (width 0.25) (layer B.Cu) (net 11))
 (segment (start 61.595 32.385) (end 61.595 33.895) (width 0.25) (layer B.Cu) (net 11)))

